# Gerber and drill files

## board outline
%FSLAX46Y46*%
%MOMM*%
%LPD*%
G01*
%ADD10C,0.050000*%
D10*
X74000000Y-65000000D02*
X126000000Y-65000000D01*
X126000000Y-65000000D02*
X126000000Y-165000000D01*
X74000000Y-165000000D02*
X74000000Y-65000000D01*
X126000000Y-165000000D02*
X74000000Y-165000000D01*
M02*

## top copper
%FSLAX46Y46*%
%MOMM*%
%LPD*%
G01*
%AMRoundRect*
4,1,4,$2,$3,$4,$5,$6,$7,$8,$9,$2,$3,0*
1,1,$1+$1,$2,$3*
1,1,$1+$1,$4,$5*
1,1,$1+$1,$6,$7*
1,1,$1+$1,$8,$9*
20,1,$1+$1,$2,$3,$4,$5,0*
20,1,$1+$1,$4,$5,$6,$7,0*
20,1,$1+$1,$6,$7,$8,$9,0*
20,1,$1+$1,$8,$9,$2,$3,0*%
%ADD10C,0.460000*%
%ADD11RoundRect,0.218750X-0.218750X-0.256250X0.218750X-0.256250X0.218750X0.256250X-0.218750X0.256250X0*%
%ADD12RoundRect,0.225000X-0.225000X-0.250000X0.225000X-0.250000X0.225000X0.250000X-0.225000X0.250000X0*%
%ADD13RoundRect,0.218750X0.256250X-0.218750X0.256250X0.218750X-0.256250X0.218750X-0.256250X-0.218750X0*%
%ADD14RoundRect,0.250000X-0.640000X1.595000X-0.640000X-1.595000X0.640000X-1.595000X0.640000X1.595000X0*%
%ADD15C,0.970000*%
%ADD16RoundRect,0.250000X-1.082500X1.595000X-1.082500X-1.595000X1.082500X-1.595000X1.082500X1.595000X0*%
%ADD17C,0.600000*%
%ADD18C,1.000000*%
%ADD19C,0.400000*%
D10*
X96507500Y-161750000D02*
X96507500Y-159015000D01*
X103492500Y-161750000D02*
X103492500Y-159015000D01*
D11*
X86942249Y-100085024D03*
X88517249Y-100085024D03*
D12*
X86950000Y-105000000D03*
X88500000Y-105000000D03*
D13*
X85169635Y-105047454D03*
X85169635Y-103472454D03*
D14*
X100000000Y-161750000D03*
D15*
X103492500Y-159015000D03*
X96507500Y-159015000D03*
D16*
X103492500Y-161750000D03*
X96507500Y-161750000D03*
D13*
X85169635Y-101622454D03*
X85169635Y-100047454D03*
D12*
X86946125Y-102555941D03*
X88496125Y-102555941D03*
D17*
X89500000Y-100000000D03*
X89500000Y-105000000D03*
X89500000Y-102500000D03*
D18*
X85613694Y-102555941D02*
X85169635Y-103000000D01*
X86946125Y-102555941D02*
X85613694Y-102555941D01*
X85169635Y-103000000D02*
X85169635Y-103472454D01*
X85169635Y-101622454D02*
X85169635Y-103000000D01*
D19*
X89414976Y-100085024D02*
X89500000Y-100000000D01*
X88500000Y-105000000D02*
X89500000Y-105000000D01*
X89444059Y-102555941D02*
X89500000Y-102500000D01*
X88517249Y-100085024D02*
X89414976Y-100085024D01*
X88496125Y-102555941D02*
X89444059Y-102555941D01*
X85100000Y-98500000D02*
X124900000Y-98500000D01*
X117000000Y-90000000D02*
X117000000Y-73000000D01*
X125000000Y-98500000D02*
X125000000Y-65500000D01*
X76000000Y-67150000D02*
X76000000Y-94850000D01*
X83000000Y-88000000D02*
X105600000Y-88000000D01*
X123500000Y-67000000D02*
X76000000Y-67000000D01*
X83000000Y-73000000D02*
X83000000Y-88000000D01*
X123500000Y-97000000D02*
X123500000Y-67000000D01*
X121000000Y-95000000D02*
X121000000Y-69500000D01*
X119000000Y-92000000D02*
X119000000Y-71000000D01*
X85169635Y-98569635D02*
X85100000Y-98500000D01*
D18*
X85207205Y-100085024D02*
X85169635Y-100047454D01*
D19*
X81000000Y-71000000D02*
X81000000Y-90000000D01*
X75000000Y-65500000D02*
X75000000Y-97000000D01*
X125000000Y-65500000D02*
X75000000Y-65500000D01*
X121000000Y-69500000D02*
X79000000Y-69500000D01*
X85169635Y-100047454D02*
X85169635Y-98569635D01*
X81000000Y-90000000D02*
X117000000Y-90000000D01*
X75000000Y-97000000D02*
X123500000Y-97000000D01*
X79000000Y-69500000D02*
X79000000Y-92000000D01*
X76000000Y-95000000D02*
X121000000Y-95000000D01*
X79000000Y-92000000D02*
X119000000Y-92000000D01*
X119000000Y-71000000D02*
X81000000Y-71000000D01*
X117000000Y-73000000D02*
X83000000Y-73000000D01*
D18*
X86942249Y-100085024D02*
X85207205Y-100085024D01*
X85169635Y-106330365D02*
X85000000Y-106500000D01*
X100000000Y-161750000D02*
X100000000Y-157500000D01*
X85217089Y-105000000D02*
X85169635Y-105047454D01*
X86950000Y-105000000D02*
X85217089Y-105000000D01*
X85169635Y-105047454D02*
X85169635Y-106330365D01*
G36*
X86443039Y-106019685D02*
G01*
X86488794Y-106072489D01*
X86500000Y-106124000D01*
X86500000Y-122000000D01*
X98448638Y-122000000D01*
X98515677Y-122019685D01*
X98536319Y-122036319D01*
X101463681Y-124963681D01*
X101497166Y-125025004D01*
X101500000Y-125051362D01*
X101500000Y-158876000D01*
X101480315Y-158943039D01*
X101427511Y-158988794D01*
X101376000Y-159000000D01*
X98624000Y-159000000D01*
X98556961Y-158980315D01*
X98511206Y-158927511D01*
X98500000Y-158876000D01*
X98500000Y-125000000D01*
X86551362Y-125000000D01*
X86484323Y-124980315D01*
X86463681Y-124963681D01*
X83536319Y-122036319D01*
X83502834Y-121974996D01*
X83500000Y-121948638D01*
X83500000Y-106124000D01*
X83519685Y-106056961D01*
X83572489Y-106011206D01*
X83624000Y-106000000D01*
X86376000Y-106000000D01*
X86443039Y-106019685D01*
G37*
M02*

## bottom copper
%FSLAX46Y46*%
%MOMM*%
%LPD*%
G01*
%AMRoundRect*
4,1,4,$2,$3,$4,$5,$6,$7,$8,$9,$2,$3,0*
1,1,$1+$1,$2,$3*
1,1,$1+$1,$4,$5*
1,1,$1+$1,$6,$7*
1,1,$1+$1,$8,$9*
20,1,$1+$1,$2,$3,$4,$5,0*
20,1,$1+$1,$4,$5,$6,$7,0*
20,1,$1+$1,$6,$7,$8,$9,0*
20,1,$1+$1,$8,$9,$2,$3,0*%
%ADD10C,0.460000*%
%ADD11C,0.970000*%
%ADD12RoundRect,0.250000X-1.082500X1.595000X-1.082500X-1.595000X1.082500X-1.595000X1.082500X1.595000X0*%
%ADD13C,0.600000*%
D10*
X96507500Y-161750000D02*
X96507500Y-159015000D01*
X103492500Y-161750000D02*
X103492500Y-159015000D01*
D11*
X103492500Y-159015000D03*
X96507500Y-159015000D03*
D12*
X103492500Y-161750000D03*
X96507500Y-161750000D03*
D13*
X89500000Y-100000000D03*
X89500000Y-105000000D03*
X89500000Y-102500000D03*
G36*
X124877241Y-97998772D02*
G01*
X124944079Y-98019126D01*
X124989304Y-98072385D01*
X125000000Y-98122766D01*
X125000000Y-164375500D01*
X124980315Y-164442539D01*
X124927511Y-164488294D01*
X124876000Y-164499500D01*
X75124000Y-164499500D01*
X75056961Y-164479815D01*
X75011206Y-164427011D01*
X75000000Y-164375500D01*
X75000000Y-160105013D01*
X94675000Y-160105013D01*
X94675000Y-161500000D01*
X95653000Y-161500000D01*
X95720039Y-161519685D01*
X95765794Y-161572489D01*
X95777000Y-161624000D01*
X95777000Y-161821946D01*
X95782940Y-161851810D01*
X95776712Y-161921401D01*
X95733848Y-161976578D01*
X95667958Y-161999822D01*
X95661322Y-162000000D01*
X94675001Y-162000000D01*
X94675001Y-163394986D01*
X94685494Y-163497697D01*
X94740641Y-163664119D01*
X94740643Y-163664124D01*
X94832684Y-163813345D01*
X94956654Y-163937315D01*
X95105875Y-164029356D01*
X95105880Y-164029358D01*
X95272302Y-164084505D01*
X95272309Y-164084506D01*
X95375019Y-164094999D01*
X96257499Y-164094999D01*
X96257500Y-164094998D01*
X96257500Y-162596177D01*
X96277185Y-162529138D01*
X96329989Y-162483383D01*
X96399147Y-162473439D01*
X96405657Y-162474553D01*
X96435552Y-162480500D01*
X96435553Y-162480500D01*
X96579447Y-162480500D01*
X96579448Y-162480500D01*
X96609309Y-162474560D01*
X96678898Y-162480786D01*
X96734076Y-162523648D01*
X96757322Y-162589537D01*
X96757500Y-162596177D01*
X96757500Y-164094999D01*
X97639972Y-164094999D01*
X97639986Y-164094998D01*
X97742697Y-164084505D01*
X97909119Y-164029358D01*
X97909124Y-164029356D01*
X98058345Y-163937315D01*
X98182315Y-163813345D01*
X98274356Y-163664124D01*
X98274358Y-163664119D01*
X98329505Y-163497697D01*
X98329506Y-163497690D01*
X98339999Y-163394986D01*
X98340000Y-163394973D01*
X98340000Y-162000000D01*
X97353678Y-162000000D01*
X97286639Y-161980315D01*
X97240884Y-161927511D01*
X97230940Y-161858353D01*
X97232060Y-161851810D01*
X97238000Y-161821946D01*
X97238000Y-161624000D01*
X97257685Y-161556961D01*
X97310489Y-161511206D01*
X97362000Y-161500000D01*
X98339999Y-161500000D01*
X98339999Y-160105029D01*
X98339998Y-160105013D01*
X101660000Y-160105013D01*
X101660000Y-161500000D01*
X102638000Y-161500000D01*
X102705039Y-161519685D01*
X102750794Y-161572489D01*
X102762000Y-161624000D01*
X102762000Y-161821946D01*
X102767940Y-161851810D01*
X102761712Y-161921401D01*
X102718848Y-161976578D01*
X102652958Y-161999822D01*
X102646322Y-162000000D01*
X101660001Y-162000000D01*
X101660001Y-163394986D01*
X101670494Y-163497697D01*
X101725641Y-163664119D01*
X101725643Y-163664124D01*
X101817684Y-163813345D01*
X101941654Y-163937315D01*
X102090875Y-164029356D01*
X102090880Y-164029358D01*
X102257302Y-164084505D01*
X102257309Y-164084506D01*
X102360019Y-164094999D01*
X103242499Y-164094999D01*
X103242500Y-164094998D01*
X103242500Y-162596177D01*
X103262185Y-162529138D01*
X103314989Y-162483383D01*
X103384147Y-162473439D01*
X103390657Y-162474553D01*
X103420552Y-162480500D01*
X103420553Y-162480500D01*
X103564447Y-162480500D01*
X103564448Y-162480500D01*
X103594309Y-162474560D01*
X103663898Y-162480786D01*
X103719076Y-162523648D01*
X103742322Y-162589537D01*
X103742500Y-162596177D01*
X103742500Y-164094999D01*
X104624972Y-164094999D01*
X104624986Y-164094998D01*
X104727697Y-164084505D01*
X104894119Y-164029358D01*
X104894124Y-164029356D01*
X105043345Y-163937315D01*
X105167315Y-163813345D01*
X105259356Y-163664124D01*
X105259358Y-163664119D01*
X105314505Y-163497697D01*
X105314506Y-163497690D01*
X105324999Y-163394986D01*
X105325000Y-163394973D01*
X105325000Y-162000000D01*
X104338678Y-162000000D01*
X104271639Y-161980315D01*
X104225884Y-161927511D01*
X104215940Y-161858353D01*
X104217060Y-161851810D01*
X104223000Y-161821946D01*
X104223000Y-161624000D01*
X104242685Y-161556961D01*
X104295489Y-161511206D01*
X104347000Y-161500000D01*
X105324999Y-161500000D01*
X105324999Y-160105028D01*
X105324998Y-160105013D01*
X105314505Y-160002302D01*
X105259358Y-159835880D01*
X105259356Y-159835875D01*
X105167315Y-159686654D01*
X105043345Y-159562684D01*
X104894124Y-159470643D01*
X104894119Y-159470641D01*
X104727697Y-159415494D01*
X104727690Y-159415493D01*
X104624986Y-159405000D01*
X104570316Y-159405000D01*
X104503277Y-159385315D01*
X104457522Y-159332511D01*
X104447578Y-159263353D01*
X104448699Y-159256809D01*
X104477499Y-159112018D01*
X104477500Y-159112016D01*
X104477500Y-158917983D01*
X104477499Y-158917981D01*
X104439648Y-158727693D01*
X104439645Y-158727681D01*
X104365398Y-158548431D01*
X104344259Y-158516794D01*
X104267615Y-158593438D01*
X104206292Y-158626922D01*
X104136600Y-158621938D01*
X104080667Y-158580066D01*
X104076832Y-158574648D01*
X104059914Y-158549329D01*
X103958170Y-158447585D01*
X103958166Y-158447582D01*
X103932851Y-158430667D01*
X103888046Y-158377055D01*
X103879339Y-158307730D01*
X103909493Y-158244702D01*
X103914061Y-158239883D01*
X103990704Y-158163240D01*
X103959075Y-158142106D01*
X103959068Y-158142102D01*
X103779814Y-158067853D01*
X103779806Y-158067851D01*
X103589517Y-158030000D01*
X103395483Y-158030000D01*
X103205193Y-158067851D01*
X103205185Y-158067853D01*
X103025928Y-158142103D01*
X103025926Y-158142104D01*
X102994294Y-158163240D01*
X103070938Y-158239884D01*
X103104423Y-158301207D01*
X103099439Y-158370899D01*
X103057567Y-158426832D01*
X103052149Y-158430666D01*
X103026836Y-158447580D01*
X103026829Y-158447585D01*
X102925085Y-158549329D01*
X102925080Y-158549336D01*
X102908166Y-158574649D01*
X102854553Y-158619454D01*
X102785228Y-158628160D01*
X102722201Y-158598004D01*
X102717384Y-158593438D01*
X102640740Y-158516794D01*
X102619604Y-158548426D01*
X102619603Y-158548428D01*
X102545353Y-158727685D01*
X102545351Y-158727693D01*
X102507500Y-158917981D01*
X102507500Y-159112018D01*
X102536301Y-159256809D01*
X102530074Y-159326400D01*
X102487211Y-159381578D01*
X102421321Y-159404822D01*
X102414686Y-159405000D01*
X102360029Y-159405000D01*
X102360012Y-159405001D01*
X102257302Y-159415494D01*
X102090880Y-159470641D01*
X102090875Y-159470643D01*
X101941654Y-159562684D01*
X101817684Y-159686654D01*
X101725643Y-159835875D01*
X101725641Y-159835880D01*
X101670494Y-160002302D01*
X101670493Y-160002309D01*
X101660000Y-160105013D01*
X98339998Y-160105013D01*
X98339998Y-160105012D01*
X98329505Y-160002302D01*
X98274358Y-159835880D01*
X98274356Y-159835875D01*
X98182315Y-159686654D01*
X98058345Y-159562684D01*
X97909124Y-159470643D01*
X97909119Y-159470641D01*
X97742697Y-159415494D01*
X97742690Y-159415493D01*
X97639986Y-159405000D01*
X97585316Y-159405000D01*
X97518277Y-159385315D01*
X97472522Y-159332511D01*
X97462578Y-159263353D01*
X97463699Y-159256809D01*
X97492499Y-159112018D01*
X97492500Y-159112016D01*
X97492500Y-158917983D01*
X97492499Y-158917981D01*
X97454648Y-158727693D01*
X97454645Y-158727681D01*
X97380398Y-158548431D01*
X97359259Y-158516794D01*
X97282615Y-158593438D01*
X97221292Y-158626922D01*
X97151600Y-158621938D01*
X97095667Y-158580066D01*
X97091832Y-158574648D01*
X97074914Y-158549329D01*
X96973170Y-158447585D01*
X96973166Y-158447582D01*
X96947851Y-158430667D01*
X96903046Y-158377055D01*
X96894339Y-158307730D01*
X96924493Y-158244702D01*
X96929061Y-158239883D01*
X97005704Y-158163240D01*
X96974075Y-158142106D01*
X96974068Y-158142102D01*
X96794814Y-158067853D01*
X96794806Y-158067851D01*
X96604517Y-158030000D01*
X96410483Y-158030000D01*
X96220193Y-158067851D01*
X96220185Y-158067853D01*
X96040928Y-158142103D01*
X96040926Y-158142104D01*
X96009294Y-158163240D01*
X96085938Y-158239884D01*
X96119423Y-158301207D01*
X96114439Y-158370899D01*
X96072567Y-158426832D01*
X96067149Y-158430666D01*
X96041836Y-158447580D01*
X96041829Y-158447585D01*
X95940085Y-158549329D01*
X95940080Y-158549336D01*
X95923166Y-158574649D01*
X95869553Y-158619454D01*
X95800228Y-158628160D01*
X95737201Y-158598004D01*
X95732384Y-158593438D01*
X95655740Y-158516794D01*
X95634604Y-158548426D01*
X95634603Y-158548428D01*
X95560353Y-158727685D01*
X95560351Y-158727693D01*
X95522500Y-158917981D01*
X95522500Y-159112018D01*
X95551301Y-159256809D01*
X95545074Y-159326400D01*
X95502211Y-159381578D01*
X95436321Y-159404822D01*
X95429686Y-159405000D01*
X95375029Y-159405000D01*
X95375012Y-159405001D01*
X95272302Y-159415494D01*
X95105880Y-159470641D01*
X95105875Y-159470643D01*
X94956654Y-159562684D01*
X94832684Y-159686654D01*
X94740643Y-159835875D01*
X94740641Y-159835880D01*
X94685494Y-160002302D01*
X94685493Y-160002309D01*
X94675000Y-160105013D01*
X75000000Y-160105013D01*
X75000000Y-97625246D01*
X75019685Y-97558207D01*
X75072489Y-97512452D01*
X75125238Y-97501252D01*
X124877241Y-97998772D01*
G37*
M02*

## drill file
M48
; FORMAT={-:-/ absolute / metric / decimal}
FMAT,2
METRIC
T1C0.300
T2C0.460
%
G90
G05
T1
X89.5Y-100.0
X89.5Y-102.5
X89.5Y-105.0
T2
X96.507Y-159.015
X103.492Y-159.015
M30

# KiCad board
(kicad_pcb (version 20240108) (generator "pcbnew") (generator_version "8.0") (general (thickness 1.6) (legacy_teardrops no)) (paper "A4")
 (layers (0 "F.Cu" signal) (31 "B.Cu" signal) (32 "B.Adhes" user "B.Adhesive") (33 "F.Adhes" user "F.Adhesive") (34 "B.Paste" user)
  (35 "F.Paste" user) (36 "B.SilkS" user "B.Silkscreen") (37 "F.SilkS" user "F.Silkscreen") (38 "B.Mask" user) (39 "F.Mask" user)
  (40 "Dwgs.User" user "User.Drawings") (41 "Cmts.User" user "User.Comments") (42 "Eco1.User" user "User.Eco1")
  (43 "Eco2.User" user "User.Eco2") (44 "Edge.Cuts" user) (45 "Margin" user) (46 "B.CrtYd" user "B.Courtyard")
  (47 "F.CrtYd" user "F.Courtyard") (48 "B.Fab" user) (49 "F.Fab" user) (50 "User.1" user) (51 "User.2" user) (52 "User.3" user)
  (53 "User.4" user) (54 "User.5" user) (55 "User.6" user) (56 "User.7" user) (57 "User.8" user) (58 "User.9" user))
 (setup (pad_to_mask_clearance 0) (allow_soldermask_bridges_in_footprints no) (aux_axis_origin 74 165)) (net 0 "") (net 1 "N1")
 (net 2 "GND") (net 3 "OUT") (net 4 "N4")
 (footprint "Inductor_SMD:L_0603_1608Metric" (layer "F.Cu") (at 87.729749 100.085024)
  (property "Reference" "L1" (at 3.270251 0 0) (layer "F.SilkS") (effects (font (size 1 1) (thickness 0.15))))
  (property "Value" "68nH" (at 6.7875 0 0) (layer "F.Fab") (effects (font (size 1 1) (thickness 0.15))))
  (pad "1" smd roundrect (at -0.7875 0) (size 0.875 0.95) (layers "F.Cu" "F.Paste" "F.Mask") (roundrect_rratio 0.25) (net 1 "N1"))
  (pad "2" smd roundrect (at 0.7875 0) (size 0.875 0.95) (layers "F.Cu" "F.Paste" "F.Mask") (roundrect_rratio 0.25) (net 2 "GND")))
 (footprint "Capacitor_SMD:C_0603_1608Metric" (layer "F.Cu") (at 87.725 105)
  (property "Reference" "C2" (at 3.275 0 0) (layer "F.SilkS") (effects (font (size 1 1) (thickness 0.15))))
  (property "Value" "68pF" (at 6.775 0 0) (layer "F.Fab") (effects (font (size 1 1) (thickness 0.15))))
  (pad "1" smd roundrect (at -0.775 0) (size 0.9 0.95) (layers "F.Cu" "F.Paste" "F.Mask") (roundrect_rratio 0.25) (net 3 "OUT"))
  (pad "2" smd roundrect (at 0.775 0) (size 0.9 0.95) (layers "F.Cu" "F.Paste" "F.Mask") (roundrect_rratio 0.25) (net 2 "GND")))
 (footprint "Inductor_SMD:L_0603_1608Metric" (layer "F.Cu") (at 85.169635 104.259954 90)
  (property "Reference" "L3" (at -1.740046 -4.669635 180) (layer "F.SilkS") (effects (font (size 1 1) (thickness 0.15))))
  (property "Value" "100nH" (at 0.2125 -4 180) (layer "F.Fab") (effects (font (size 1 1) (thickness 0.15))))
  (pad "1" smd roundrect (at -0.7875 0 90) (size 0.875 0.95) (layers "F.Cu" "F.Paste" "F.Mask") (roundrect_rratio 0.25) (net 3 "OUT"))
  (pad "2" smd roundrect (at 0.7875 0 90) (size 0.875 0.95) (layers "F.Cu" "F.Paste" "F.Mask") (roundrect_rratio 0.25) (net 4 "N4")))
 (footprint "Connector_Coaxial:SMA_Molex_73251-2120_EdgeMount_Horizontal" (layer "F.Cu") (at 100 162 -90)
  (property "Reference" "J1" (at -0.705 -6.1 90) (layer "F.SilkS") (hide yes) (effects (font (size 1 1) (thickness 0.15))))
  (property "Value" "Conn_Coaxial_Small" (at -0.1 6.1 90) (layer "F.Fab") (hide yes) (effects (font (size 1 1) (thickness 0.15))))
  (fp_line (start -0.25 3.4925) (end -2.985 3.4925) (stroke (width 0.46) (type default)) (layer "F.Cu"))
  (fp_line (start -0.25 -3.4925) (end -2.985 -3.4925) (stroke (width 0.46) (type default)) (layer "F.Cu"))
  (fp_line (start -0.25 3.4925) (end -2.985 3.4925) (stroke (width 0.46) (type default)) (layer "B.Cu"))
  (fp_line (start -0.25 -3.4925) (end -2.985 -3.4925) (stroke (width 0.46) (type default)) (layer "B.Cu"))
  (pad "1" smd roundrect (at -0.25 0 270) (size 3.69 1.78) (layers "F.Cu" "F.Paste" "F.Mask") (roundrect_rratio 0.1404494382) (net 3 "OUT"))
  (pad "2" thru_hole circle (at -2.985 -3.4925 270) (size 0.97 0.97) (drill 0.46) (layers "*.Cu") (remove_unused_layers no) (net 2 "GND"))
  (pad "2" thru_hole circle (at -2.985 3.4925 270) (size 0.97 0.97) (drill 0.46) (layers "*.Cu") (remove_unused_layers no) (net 2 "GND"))
  (pad "2" smd roundrect (at -0.25 -3.4925 270) (size 3.69 2.665) (layers "F.Cu" "F.Paste" "F.Mask") (roundrect_rratio 0.09380863039)
   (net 2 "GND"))
  (pad "2" smd roundrect (at -0.25 -3.4925 270) (size 3.69 2.665) (layers "B.Cu" "B.Paste" "B.Mask") (roundrect_rratio 0.09380863039)
   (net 2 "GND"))
  (pad "2" smd roundrect (at -0.25 3.4925 270) (size 3.69 2.665) (layers "F.Cu" "F.Paste" "F.Mask") (roundrect_rratio 0.09380863039)
   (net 2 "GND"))
  (pad "2" smd roundrect (at -0.25 3.4925 270) (size 3.69 2.665) (layers "B.Cu" "B.Paste" "B.Mask") (roundrect_rratio 0.09380863039)
   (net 2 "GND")))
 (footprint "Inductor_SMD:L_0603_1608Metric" (layer "F.Cu") (at 85.169635 100.834954 90)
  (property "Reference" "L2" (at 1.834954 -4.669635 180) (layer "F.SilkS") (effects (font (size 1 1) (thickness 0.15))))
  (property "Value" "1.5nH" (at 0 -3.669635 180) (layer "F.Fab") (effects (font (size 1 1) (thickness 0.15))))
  (pad "1" smd roundrect (at -0.7875 0 90) (size 0.875 0.95) (layers "F.Cu" "F.Paste" "F.Mask") (roundrect_rratio 0.25) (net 4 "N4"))
  (pad "2" smd roundrect (at 0.7875 0 90) (size 0.875 0.95) (layers "F.Cu" "F.Paste" "F.Mask") (roundrect_rratio 0.25) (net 1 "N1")))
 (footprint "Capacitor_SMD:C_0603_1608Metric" (layer "F.Cu") (at 87.721125 102.555941)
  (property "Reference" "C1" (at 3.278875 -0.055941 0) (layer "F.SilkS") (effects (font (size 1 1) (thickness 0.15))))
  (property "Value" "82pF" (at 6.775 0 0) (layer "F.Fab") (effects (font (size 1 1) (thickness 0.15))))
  (pad "1" smd roundrect (at -0.775 0) (size 0.9 0.95) (layers "F.Cu" "F.Paste" "F.Mask") (roundrect_rratio 0.25) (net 4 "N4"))
  (pad "2" smd roundrect (at 0.775 0) (size 0.9 0.95) (layers "F.Cu" "F.Paste" "F.Mask") (roundrect_rratio 0.25) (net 2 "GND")))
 (gr_line (start 74 65) (end 126 65) (stroke (width 0.05) (type default)) (layer "Edge.Cuts"))
 (gr_line (start 126 65) (end 126 165) (stroke (width 0.05) (type default)) (layer "Edge.Cuts"))
 (gr_line (start 74 165) (end 74 65) (stroke (width 0.05) (type default)) (layer "Edge.Cuts"))
 (gr_line (start 126 165) (end 74 165) (stroke (width 0.05) (type default)) (layer "Edge.Cuts"))
 (segment (start 85.613694 102.555941) (end 85.169635 103) (width 1) (layer "F.Cu") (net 4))
 (segment (start 86.946125 102.555941) (end 85.613694 102.555941) (width 1) (layer "F.Cu") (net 4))
 (segment (start 85.169635 103) (end 85.169635 103.472454) (width 1) (layer "F.Cu") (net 4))
 (segment (start 85.169635 101.622454) (end 85.169635 103) (width 1) (layer "F.Cu") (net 4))
 (segment (start 89.414976 100.085024) (end 89.5 100) (width 0.4) (layer "F.Cu") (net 2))
 (segment (start 88.5 105) (end 89.5 105) (width 0.4) (layer "F.Cu") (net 2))
 (segment (start 89.444059 102.555941) (end 89.5 102.5) (width 0.4) (layer "F.Cu") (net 2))
 (segment (start 88.517249 100.085024) (end 89.414976 100.085024) (width 0.4) (layer "F.Cu") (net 2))
 (segment (start 88.496125 102.555941) (end 89.444059 102.555941) (width 0.4) (layer "F.Cu") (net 2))
 (via (at 89.5 100) (size 0.6) (drill 0.3) (layers "F.Cu" "B.Cu") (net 2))
 (via (at 89.5 105) (size 0.6) (drill 0.3) (layers "F.Cu" "B.Cu") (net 2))
 (via (at 89.5 102.5) (size 0.6) (drill 0.3) (layers "F.Cu" "B.Cu") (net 2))
 (segment (start 85.1 98.5) (end 124.9 98.5) (width 0.4) (layer "F.Cu") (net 1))
 (segment (start 117 90) (end 117 73) (width 0.4) (layer "F.Cu") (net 1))
 (segment (start 125 98.5) (end 125 65.5) (width 0.4) (layer "F.Cu") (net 1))
 (segment (start 76 67.15) (end 76 94.85) (width 0.4) (layer "F.Cu") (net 1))
 (segment (start 83 88) (end 105.6 88) (width 0.4) (layer "F.Cu") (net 1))
 (segment (start 123.5 67) (end 76 67) (width 0.4) (layer "F.Cu") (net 1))
 (segment (start 83 73) (end 83 88) (width 0.4) (layer "F.Cu") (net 1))
 (segment (start 123.5 97) (end 123.5 67) (width 0.4) (layer "F.Cu") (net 1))
 (segment (start 121 95) (end 121 69.5) (width 0.4) (layer "F.Cu") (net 1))
 (segment (start 119 92) (end 119 71) (width 0.4) (layer "F.Cu") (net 1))
 (segment (start 85.169635 98.569635) (end 85.1 98.5) (width 0.4) (layer "F.Cu") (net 1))
 (segment (start 85.207205 100.085024) (end 85.169635 100.047454) (width 1) (layer "F.Cu") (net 1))
 (segment (start 81 71) (end 81 90) (width 0.4) (layer "F.Cu") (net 1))
 (segment (start 75 65.5) (end 75 97) (width 0.4) (layer "F.Cu") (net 1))
 (segment (start 125 65.5) (end 75 65.5) (width 0.4) (layer "F.Cu") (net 1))
 (segment (start 121 69.5) (end 79 69.5) (width 0.4) (layer "F.Cu") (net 1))
 (segment (start 85.169635 100.047454) (end 85.169635 98.569635) (width 0.4) (layer "F.Cu") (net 1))
 (segment (start 81 90) (end 117 90) (width 0.4) (layer "F.Cu") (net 1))
 (segment (start 75 97) (end 123.5 97) (width 0.4) (layer "F.Cu") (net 1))
 (segment (start 79 69.5) (end 79 92) (width 0.4) (layer "F.Cu") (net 1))
 (segment (start 76 95) (end 121 95) (width 0.4) (layer "F.Cu") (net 1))
 (segment (start 79 92) (end 119 92) (width 0.4) (layer "F.Cu") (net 1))
 (segment (start 119 71) (end 81 71) (width 0.4) (layer "F.Cu") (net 1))
 (segment (start 117 73) (end 83 73) (width 0.4) (layer "F.Cu") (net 1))
 (segment (start 86.942249 100.085024) (end 85.207205 100.085024) (width 1) (layer "F.Cu") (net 1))
 (segment (start 85.169635 106.330365) (end 85 106.5) (width 1) (layer "F.Cu") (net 3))
 (segment (start 100 161.75) (end 100 157.5) (width 1) (layer "F.Cu") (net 3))
 (segment (start 85.217089 105) (end 85.169635 105.047454) (width 1) (layer "F.Cu") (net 3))
 (segment (start 86.95 105) (end 85.217089 105) (width 1) (layer "F.Cu") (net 3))
 (segment (start 85.169635 105.047454) (end 85.169635 106.330365) (width 1) (layer "F.Cu") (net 3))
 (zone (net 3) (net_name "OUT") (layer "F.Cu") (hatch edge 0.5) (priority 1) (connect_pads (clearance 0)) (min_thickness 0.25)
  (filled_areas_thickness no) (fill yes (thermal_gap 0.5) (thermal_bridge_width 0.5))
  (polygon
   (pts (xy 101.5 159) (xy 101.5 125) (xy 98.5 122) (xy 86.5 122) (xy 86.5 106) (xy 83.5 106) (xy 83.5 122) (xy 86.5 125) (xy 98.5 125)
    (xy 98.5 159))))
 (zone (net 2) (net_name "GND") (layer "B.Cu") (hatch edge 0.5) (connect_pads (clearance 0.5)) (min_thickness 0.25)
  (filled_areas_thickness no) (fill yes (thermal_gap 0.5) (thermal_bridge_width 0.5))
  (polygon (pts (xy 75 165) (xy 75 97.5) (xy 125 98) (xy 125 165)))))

